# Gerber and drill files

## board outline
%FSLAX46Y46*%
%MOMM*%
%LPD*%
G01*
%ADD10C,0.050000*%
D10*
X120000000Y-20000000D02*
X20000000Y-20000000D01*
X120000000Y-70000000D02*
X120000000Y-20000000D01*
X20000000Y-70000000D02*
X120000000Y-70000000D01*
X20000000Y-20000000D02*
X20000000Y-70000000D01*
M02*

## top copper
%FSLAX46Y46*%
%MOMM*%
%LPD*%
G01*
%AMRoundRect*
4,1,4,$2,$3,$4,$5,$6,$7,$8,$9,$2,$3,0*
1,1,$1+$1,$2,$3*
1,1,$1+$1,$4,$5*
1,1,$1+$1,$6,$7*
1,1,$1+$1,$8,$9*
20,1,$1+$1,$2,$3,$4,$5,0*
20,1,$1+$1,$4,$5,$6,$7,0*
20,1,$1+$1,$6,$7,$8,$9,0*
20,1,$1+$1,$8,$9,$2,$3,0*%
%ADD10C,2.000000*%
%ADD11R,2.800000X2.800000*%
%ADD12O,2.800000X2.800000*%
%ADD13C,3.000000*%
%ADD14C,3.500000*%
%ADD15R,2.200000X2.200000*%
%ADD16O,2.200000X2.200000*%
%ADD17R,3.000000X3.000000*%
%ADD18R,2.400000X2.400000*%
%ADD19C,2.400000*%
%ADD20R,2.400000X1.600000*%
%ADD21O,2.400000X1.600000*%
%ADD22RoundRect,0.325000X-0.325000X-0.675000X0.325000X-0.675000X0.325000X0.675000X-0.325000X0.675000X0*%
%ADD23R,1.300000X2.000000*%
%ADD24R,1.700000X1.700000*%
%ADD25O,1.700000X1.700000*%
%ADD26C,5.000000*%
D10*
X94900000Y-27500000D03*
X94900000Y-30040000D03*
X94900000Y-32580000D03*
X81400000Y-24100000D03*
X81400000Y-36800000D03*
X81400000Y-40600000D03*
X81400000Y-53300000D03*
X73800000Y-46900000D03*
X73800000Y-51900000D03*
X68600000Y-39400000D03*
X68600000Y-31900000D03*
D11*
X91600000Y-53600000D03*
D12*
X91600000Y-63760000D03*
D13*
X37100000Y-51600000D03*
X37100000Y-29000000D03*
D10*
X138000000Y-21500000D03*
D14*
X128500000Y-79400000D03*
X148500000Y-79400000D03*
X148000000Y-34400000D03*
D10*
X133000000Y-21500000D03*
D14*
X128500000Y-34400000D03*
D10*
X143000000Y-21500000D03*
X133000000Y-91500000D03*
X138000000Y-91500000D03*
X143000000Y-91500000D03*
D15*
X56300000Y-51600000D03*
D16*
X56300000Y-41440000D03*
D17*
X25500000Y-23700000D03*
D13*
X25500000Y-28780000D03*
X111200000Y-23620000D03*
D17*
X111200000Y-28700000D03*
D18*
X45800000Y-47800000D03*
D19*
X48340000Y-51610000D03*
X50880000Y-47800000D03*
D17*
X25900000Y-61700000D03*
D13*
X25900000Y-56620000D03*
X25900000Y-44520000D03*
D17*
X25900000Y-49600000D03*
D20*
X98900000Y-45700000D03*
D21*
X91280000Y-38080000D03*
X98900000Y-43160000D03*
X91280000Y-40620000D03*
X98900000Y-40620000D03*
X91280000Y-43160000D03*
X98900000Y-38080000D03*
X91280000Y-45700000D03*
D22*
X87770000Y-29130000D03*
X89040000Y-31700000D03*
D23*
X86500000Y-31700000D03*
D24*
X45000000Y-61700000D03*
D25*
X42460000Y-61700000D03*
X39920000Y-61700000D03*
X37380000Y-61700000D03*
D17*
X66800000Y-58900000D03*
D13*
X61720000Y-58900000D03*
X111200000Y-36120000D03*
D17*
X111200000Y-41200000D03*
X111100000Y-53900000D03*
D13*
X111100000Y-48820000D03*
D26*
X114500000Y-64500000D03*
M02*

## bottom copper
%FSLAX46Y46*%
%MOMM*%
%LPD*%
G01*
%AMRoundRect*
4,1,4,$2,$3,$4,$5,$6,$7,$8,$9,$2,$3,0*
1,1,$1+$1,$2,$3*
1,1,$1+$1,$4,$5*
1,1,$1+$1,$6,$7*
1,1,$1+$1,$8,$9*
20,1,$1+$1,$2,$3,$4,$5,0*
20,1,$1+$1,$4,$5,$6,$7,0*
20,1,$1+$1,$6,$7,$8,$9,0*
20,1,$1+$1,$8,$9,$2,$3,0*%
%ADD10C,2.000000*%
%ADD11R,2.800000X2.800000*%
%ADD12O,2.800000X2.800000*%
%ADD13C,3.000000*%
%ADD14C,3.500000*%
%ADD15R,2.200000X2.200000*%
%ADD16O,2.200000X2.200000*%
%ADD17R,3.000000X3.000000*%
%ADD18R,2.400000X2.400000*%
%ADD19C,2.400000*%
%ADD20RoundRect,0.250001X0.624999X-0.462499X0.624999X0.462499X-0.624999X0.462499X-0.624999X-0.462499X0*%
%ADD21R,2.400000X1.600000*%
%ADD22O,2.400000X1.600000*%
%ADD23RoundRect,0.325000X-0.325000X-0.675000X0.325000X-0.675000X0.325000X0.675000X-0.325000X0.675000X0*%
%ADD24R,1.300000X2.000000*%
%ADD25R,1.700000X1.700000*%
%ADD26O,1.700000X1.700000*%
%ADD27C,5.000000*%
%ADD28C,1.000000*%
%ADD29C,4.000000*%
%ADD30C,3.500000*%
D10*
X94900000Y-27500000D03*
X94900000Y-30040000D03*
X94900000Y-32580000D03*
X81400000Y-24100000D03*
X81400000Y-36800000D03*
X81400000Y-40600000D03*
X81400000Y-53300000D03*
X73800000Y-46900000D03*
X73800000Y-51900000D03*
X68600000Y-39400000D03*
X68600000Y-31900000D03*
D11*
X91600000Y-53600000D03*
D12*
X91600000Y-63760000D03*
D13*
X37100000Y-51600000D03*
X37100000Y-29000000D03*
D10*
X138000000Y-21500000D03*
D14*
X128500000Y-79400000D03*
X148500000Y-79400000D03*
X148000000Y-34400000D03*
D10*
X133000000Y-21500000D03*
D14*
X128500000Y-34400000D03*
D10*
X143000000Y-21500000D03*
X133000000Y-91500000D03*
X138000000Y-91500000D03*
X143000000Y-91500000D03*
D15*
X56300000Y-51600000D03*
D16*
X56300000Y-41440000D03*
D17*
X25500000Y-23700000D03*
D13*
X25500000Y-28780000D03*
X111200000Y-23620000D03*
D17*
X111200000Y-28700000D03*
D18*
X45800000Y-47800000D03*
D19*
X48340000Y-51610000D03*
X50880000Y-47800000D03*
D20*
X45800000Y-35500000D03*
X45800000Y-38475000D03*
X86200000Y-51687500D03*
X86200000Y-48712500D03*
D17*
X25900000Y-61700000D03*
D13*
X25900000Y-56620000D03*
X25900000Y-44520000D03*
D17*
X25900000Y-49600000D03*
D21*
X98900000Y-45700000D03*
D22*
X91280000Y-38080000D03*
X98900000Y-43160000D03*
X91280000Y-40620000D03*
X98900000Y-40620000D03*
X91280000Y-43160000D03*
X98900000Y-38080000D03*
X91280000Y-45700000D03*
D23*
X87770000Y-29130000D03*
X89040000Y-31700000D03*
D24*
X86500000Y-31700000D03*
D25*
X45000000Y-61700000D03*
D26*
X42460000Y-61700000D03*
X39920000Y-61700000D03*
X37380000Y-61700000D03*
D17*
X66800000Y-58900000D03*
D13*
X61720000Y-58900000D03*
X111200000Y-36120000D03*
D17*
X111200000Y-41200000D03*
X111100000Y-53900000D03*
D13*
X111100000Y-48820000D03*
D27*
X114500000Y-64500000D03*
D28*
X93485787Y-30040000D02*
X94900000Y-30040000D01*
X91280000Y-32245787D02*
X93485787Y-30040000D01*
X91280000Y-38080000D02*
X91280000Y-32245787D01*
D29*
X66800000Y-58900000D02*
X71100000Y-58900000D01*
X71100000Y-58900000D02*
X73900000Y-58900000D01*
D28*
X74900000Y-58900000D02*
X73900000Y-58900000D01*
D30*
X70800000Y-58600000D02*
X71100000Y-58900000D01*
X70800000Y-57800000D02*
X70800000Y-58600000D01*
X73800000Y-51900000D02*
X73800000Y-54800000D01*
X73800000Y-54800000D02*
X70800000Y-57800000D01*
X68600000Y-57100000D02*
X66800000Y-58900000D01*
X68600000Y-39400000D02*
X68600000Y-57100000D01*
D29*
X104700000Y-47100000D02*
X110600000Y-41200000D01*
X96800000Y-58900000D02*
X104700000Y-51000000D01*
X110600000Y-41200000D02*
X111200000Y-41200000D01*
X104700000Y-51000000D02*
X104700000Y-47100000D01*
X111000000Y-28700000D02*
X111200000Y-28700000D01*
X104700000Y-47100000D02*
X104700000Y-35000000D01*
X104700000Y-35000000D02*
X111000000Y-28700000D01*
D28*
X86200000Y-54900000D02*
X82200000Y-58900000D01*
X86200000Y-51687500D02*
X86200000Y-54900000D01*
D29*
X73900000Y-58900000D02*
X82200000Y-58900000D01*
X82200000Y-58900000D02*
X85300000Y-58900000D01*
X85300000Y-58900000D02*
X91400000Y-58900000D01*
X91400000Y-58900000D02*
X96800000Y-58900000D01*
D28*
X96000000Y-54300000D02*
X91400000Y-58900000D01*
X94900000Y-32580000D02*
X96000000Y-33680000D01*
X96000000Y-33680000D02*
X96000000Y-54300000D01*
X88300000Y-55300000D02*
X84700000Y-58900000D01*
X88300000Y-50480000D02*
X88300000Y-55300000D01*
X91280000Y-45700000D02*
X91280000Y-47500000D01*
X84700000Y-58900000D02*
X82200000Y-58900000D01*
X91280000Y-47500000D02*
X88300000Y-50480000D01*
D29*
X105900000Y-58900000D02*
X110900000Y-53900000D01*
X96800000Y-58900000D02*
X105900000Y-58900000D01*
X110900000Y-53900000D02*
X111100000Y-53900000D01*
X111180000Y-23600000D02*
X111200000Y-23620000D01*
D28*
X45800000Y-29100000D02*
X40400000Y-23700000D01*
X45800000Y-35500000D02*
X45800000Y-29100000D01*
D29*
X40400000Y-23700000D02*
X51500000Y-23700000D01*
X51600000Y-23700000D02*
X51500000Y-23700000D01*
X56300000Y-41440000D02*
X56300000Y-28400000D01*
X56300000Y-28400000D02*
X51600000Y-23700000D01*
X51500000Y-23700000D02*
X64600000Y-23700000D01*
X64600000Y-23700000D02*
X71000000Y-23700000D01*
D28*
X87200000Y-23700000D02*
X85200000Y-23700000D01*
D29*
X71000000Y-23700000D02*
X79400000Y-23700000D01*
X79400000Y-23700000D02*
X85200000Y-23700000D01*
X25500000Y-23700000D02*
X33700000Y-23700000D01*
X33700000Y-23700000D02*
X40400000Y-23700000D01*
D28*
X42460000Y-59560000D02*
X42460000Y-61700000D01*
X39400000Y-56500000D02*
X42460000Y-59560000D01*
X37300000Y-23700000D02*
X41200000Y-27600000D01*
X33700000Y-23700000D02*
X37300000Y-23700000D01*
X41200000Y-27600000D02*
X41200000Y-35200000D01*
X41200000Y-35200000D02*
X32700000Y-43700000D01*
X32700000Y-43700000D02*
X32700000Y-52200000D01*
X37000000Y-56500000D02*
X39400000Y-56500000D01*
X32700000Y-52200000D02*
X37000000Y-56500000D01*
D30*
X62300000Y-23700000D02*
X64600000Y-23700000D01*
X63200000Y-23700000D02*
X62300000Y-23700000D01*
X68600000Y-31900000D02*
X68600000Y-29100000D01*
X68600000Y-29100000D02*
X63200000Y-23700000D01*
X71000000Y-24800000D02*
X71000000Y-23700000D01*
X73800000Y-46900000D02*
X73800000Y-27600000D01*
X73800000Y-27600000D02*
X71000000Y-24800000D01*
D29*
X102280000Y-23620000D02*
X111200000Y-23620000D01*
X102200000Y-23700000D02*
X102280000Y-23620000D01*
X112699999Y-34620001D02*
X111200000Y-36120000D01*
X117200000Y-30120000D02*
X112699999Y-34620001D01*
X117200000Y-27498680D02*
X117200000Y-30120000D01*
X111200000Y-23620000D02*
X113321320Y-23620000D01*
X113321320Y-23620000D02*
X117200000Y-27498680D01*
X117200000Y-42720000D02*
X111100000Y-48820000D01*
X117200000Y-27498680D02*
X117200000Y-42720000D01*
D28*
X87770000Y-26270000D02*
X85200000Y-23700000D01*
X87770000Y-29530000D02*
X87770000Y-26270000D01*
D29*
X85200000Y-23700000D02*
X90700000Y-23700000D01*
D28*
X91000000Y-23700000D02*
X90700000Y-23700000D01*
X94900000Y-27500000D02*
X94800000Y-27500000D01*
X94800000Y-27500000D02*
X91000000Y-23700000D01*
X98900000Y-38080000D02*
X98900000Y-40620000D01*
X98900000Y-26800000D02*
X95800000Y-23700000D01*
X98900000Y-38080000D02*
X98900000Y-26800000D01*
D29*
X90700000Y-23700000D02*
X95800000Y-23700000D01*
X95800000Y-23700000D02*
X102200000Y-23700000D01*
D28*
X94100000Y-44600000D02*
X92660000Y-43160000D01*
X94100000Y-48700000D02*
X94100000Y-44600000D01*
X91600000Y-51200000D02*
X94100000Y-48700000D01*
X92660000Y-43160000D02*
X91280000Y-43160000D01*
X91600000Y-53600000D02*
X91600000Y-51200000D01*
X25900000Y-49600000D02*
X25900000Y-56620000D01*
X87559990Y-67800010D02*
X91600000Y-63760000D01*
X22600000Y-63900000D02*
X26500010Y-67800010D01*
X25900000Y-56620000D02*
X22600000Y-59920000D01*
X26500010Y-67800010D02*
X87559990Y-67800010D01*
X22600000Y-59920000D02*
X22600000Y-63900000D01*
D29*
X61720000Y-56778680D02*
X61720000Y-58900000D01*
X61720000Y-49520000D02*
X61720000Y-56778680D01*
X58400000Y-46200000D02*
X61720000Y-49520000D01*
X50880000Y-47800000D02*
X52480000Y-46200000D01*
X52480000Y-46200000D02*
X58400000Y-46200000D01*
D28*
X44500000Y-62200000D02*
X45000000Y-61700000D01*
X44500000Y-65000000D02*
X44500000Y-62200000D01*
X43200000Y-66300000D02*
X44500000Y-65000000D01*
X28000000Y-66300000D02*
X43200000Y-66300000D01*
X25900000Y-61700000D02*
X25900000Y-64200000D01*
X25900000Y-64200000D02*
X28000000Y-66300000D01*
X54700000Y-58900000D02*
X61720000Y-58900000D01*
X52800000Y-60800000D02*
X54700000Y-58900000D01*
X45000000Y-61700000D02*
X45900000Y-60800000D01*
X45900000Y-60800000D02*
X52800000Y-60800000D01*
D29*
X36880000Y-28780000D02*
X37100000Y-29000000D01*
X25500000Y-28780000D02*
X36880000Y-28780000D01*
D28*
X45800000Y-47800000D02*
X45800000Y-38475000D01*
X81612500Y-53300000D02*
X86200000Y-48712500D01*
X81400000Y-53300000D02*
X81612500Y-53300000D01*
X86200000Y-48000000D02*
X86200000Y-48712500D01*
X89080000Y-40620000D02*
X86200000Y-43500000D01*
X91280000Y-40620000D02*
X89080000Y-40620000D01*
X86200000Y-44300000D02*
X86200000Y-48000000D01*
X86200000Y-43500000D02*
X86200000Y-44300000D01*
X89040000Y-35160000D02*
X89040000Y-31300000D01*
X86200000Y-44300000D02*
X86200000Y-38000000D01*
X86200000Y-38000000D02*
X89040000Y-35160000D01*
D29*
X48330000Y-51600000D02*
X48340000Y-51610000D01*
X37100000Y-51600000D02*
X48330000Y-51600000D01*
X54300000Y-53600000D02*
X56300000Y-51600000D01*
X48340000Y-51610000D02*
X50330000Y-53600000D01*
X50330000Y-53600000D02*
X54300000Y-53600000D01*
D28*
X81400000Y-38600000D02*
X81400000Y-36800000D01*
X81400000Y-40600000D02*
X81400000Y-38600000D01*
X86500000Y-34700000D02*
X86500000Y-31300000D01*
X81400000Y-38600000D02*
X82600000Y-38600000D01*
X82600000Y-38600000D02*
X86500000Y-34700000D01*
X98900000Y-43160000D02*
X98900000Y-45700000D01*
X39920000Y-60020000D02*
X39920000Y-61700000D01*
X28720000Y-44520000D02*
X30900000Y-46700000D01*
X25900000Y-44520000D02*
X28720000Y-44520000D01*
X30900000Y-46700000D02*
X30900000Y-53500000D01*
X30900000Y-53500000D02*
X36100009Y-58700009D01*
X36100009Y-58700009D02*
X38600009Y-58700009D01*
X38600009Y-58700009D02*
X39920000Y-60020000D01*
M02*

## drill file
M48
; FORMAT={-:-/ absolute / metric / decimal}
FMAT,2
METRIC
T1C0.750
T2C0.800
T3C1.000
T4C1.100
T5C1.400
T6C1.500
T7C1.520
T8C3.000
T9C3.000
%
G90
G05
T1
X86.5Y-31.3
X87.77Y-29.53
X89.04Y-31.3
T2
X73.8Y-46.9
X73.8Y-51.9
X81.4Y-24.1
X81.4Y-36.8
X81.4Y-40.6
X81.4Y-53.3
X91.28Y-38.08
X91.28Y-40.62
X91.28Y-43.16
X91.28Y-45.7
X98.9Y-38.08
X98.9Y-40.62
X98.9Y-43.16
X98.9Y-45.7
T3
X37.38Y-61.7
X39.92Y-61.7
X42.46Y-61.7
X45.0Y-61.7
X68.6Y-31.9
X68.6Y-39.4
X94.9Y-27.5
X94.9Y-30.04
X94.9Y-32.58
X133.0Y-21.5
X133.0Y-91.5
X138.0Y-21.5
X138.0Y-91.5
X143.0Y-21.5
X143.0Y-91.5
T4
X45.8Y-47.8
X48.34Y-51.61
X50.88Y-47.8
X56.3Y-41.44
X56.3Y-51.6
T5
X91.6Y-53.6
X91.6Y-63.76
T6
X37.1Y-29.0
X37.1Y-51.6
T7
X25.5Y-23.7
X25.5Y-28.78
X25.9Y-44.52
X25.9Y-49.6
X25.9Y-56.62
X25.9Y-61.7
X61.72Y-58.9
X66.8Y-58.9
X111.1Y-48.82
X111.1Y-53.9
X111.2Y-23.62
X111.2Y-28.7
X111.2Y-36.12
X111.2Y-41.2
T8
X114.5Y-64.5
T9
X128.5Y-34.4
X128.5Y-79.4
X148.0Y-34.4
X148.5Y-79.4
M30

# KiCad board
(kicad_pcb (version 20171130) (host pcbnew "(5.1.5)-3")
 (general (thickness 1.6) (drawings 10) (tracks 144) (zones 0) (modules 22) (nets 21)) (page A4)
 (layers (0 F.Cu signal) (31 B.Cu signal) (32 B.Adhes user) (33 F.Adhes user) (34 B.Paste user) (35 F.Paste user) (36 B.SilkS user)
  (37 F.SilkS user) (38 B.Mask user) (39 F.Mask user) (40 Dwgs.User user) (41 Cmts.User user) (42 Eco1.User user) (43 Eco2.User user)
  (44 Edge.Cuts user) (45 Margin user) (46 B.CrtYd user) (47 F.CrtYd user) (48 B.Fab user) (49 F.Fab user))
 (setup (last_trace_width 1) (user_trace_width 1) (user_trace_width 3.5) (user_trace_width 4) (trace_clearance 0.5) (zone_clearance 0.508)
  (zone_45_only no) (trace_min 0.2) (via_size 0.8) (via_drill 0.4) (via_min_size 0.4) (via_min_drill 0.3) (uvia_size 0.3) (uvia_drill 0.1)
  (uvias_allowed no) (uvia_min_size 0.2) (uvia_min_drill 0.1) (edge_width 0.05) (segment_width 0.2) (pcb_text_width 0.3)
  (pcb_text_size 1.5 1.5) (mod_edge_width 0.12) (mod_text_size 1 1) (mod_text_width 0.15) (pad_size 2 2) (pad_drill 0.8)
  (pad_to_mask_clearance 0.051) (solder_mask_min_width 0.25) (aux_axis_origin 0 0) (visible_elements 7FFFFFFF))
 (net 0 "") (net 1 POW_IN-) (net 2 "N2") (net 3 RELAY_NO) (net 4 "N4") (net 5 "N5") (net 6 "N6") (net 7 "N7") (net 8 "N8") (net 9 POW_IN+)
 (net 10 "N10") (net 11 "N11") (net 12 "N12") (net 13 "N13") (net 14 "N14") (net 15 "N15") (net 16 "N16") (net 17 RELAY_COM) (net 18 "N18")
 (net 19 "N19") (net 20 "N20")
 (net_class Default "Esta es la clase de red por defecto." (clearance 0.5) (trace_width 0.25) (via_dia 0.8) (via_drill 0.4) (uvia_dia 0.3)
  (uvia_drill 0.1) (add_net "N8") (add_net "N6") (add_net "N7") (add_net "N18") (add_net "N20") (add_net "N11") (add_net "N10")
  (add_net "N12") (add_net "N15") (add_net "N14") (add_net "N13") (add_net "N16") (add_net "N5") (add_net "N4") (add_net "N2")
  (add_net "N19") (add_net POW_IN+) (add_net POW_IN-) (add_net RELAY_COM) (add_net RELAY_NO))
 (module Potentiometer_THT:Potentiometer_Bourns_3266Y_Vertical (layer F.Cu) (at 94.9 27.5 90)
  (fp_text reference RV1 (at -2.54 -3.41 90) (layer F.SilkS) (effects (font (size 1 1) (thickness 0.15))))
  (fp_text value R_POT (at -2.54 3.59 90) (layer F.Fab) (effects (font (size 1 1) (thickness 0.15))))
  (pad 1 thru_hole circle (at 0 0 90) (size 2 2) (drill 1) (layers *.Cu *.Mask) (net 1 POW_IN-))
  (pad 2 thru_hole circle (at -2.54 0 90) (size 2 2) (drill 1) (layers *.Cu *.Mask) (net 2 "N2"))
  (pad 3 thru_hole circle (at -5.08 0 90) (size 2 2) (drill 1) (layers *.Cu *.Mask) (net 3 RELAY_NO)))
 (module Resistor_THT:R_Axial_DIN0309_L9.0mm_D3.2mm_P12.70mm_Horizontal (layer F.Cu) (at 81.4 36.8 90)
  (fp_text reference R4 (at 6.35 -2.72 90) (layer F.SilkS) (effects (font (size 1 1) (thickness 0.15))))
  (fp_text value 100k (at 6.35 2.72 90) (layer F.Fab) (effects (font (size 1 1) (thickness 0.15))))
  (pad 2 thru_hole circle (at 12.7 0 90) (size 2 2) (drill 0.8) (layers *.Cu *.Mask) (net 1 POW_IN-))
  (pad 1 thru_hole circle (at 0 0 90) (size 2 2) (drill 0.8) (layers *.Cu *.Mask) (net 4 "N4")))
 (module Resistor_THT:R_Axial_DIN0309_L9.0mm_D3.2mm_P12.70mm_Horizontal (layer F.Cu) (at 81.4 53.3 90)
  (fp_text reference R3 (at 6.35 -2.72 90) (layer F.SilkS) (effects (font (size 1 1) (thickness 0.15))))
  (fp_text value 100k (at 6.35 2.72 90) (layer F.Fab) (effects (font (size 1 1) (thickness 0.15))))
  (pad 2 thru_hole circle (at 12.7 0 90) (size 2 2) (drill 0.8) (layers *.Cu *.Mask) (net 4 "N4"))
  (pad 1 thru_hole circle (at 0 0 90) (size 2 2) (drill 0.8) (layers *.Cu *.Mask) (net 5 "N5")))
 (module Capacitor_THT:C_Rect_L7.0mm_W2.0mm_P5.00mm (layer B.Cu) (at 73.8 51.9 90)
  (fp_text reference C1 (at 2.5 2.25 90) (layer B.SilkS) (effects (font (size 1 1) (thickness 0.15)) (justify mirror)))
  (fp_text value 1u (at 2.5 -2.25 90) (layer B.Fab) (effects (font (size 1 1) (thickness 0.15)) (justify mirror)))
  (pad 2 thru_hole circle (at 5 0 90) (size 2 2) (drill 0.8) (layers *.Cu *.Mask) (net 1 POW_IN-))
  (pad 1 thru_hole circle (at 0 0 90) (size 2 2) (drill 0.8) (layers *.Cu *.Mask) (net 3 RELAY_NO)))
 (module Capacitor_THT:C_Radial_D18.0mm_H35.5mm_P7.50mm (layer F.Cu) (at 68.6 39.4 90)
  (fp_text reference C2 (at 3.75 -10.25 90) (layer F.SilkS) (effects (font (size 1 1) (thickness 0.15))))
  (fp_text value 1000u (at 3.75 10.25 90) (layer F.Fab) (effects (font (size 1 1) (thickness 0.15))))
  (pad 1 thru_hole circle (at 0 0 90) (size 2 2) (drill 1) (layers *.Cu *.Mask) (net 3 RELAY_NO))
  (pad 2 thru_hole circle (at 7.5 0 90) (size 2 2) (drill 1) (layers *.Cu *.Mask) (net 1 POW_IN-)))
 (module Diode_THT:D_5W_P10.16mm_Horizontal (layer F.Cu) (at 91.6 53.6 270)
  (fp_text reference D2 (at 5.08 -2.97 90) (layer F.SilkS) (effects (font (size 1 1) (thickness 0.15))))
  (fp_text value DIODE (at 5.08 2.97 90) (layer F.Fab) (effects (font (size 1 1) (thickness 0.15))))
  (pad 1 thru_hole rect (at 0 0 270) (size 2.8 2.8) (drill 1.4) (layers *.Cu *.Mask) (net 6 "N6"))
  (pad 2 thru_hole oval (at 10.16 0 270) (size 2.8 2.8) (drill 1.4) (layers *.Cu *.Mask) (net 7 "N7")))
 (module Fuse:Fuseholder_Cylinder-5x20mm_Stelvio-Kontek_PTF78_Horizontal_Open (layer F.Cu) (at 37.1 51.6 90)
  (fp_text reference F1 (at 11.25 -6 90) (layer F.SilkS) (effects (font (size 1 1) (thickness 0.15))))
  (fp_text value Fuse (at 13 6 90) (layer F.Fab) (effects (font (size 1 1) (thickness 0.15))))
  (pad 1 thru_hole circle (at 0 0 90) (size 3 3) (drill 1.5) (layers *.Cu *.Mask) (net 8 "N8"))
  (pad 2 thru_hole circle (at 22.6 0 90) (size 3 3) (drill 1.5) (layers *.Cu *.Mask) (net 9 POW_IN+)))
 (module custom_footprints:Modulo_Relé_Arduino (layer F.Cu) (at 128.5 34.4 90)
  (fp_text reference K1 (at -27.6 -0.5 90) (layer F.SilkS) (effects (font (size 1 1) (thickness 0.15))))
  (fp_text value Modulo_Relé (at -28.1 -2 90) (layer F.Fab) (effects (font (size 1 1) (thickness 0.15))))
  (pad 2 thru_hole circle (at 12.9 9.5 90) (size 2 2) (drill 1) (layers *.Cu *.Mask) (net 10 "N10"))
  (pad "" np_thru_hole circle (at -45 0 90) (size 3.5 3.5) (drill 3) (layers *.Cu *.Mask))
  (pad "" np_thru_hole circle (at -45 20 90) (size 3.5 3.5) (drill 3) (layers *.Cu *.Mask))
  (pad "" np_thru_hole circle (at 0 19.5 90) (size 3.5 3.5) (drill 3) (layers *.Cu *.Mask))
  (pad 1 thru_hole circle (at 12.9 4.5 90) (size 2 2) (drill 1) (layers *.Cu *.Mask) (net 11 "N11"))
  (pad "" np_thru_hole circle (at 0 0 90) (size 3.5 3.5) (drill 3) (layers *.Cu *.Mask))
  (pad 3 thru_hole circle (at 12.9 14.5 90) (size 2 2) (drill 1) (layers *.Cu *.Mask) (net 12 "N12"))
  (pad 6 thru_hole circle (at -57.1 4.5 90) (size 2 2) (drill 1) (layers *.Cu *.Mask) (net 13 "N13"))
  (pad 5 thru_hole circle (at -57.1 9.5 90) (size 2 2) (drill 1) (layers *.Cu *.Mask) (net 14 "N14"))
  (pad 4 thru_hole circle (at -57.1 14.5 90) (size 2 2) (drill 1) (layers *.Cu *.Mask) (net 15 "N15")))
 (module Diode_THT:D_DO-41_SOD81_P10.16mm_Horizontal (layer F.Cu) (at 56.3 51.6 90)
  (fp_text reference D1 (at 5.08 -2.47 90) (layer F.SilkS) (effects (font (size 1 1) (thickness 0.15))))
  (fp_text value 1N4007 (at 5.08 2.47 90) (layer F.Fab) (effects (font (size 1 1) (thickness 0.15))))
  (pad 1 thru_hole rect (at 0 0 90) (size 2.2 2.2) (drill 1.1) (layers *.Cu *.Mask) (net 8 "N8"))
  (pad 2 thru_hole oval (at 10.16 0 90) (size 2.2 2.2) (drill 1.1) (layers *.Cu *.Mask) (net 1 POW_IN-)))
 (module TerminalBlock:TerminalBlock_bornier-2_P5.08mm (layer F.Cu) (at 25.5 23.7 270)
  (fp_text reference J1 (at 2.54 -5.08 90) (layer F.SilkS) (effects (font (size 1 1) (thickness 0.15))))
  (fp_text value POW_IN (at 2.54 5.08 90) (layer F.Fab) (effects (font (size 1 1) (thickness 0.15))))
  (pad 1 thru_hole rect (at 0 0 270) (size 3 3) (drill 1.52) (layers *.Cu *.Mask) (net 1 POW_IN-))
  (pad 2 thru_hole circle (at 5.08 0 270) (size 3 3) (drill 1.52) (layers *.Cu *.Mask) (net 9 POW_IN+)))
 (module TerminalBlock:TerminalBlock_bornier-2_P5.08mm (layer F.Cu) (at 111.2 28.7 90)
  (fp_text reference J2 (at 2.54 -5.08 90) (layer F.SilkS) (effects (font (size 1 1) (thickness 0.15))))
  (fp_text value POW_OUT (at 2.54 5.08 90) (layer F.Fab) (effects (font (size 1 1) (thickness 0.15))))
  (pad 2 thru_hole circle (at 5.08 0 90) (size 3 3) (drill 1.52) (layers *.Cu *.Mask) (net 1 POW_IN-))
  (pad 1 thru_hole rect (at 0 0 90) (size 3 3) (drill 1.52) (layers *.Cu *.Mask) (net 3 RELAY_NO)))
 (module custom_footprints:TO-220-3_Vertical (layer F.Cu) (at 45.8 47.8)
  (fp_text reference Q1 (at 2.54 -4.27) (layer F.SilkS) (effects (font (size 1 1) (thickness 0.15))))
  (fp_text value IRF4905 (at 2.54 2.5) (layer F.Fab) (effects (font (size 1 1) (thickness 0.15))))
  (pad 1 thru_hole rect (at 0 0) (size 2.4 2.4) (drill 1.1) (layers *.Cu *.Mask) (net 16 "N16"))
  (pad 2 thru_hole circle (at 2.54 3.81) (size 2.4 2.4) (drill 1.1) (layers *.Cu *.Mask) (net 8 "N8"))
  (pad 3 thru_hole circle (at 5.08 0) (size 2.4 2.4) (drill 1.1) (layers *.Cu *.Mask) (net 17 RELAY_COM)))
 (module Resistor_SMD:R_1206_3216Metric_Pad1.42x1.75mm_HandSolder (layer B.Cu) (at 45.8 36.9875 90)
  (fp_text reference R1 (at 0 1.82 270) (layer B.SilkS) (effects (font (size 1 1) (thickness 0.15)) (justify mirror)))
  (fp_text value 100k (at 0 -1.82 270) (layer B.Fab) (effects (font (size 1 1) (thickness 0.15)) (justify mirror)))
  (pad 2 smd roundrect (at 1.4875 0 90) (size 1.425 1.75) (layers B.Cu B.Paste B.Mask) (roundrect_rratio 0.175439) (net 1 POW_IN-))
  (pad 1 smd roundrect (at -1.4875 0 90) (size 1.425 1.75) (layers B.Cu B.Paste B.Mask) (roundrect_rratio 0.175439) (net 16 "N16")))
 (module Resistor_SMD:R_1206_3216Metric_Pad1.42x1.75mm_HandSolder (layer B.Cu) (at 86.2 50.2 90)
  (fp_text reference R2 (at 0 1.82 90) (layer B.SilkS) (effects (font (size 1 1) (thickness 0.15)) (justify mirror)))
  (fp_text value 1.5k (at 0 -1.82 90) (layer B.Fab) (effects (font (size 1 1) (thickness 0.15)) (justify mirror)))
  (pad 1 smd roundrect (at -1.4875 0 90) (size 1.425 1.75) (layers B.Cu B.Paste B.Mask) (roundrect_rratio 0.175439) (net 3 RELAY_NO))
  (pad 2 smd roundrect (at 1.4875 0 90) (size 1.425 1.75) (layers B.Cu B.Paste B.Mask) (roundrect_rratio 0.175439) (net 5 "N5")))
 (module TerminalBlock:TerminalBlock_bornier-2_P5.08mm (layer F.Cu) (at 25.9 61.7 90)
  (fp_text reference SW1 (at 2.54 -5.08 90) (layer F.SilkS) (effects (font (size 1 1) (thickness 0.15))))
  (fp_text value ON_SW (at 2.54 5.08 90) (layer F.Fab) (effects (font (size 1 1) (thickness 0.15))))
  (pad 1 thru_hole rect (at 0 0 90) (size 3 3) (drill 1.52) (layers *.Cu *.Mask) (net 17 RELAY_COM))
  (pad 2 thru_hole circle (at 5.08 0 90) (size 3 3) (drill 1.52) (layers *.Cu *.Mask) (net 7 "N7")))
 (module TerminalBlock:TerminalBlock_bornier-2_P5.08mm (layer F.Cu) (at 25.9 49.6 90)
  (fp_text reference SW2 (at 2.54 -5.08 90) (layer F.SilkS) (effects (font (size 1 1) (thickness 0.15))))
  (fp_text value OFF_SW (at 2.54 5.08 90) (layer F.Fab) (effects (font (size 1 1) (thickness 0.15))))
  (pad 2 thru_hole circle (at 5.08 0 90) (size 3 3) (drill 1.52) (layers *.Cu *.Mask) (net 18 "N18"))
  (pad 1 thru_hole rect (at 0 0 90) (size 3 3) (drill 1.52) (layers *.Cu *.Mask) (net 7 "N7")))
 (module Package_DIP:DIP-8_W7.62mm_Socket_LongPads (layer F.Cu) (at 98.9 45.7 180)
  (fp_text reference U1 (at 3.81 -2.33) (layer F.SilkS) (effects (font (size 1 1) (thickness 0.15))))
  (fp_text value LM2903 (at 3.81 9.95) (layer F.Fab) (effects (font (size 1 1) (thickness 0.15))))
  (pad 1 thru_hole rect (at 0 0 180) (size 2.4 1.6) (drill 0.8) (layers *.Cu *.Mask) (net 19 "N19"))
  (pad 5 thru_hole oval (at 7.62 7.62 180) (size 2.4 1.6) (drill 0.8) (layers *.Cu *.Mask) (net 2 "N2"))
  (pad 2 thru_hole oval (at 0 2.54 180) (size 2.4 1.6) (drill 0.8) (layers *.Cu *.Mask) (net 19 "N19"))
  (pad 6 thru_hole oval (at 7.62 5.08 180) (size 2.4 1.6) (drill 0.8) (layers *.Cu *.Mask) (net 5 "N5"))
  (pad 3 thru_hole oval (at 0 5.08 180) (size 2.4 1.6) (drill 0.8) (layers *.Cu *.Mask) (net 1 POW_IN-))
  (pad 7 thru_hole oval (at 7.62 2.54 180) (size 2.4 1.6) (drill 0.8) (layers *.Cu *.Mask) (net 6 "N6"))
  (pad 4 thru_hole oval (at 0 7.62 180) (size 2.4 1.6) (drill 0.8) (layers *.Cu *.Mask) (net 1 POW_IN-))
  (pad 8 thru_hole oval (at 7.62 0 180) (size 2.4 1.6) (drill 0.8) (layers *.Cu *.Mask) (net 3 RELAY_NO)))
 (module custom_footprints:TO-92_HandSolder (layer F.Cu) (at 86.5 30.8)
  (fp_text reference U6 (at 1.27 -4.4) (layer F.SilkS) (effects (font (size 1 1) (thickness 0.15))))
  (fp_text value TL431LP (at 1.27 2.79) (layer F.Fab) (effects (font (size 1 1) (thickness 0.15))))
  (pad 2 thru_hole roundrect (at 1.27 -1.27) (size 1.3 2) (drill 0.75 (offset 0 -0.4)) (layers *.Cu *.Mask) (roundrect_rratio 0.25)
   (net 1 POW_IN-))
  (pad 3 thru_hole roundrect (at 2.54 0.5) (size 1.3 2) (drill 0.75 (offset 0 0.4)) (layers *.Cu *.Mask) (roundrect_rratio 0.25)
   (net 5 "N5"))
  (pad 1 thru_hole rect (at 0 0.5) (size 1.3 2) (drill 0.75 (offset 0 0.4)) (layers *.Cu *.Mask) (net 4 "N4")))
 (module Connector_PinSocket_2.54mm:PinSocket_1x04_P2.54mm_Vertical (layer F.Cu) (at 45 61.7 270)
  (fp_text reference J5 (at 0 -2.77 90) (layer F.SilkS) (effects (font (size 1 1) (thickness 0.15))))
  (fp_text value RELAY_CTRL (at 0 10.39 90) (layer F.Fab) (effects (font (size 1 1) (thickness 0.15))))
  (pad 1 thru_hole rect (at 0 0 270) (size 1.7 1.7) (drill 1) (layers *.Cu *.Mask) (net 17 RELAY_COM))
  (pad 2 thru_hole oval (at 0 2.54 270) (size 1.7 1.7) (drill 1) (layers *.Cu *.Mask) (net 1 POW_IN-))
  (pad 3 thru_hole oval (at 0 5.08 270) (size 1.7 1.7) (drill 1) (layers *.Cu *.Mask) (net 18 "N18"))
  (pad 4 thru_hole oval (at 0 7.62 270) (size 1.7 1.7) (drill 1) (layers *.Cu *.Mask) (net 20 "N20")))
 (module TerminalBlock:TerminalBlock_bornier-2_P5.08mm (layer F.Cu) (at 66.8 58.9 180)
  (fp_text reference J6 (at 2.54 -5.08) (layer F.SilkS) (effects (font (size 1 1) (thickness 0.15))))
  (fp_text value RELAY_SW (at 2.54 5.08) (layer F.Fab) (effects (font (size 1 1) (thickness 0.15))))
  (pad 1 thru_hole rect (at 0 0 180) (size 3 3) (drill 1.52) (layers *.Cu *.Mask) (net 3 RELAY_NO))
  (pad 2 thru_hole circle (at 5.08 0 180) (size 3 3) (drill 1.52) (layers *.Cu *.Mask) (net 17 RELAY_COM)))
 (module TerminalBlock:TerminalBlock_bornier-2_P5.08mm (layer F.Cu) (at 111.2 41.2 90)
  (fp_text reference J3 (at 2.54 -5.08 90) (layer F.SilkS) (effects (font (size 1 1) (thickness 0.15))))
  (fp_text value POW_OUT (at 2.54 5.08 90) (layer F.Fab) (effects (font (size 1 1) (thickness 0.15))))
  (pad 2 thru_hole circle (at 5.08 0 90) (size 3 3) (drill 1.52) (layers *.Cu *.Mask) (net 1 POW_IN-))
  (pad 1 thru_hole rect (at 0 0 90) (size 3 3) (drill 1.52) (layers *.Cu *.Mask) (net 3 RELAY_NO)))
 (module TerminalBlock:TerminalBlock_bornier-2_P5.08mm (layer F.Cu) (at 111.1 53.9 90)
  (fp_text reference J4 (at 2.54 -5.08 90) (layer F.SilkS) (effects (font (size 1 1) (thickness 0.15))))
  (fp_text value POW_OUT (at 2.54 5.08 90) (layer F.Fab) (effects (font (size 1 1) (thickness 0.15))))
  (pad 1 thru_hole rect (at 0 0 90) (size 3 3) (drill 1.52) (layers *.Cu *.Mask) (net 3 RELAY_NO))
  (pad 2 thru_hole circle (at 5.08 0 90) (size 3 3) (drill 1.52) (layers *.Cu *.Mask) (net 1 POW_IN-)))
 (gr_line (start 120 20) (end 20 20) (layer Edge.Cuts) (width 0.05))
 (gr_line (start 120 70) (end 120 20) (layer Edge.Cuts) (width 0.05))
 (gr_line (start 20 70) (end 120 70) (layer Edge.Cuts) (width 0.05))
 (gr_line (start 20 20) (end 20 70) (layer Edge.Cuts) (width 0.05))
 (via (at 114.5 64.5) (size 5) (drill 3) (layers F.Cu B.Cu) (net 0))
 (segment (start 93.485787 30.04) (end 94.9 30.04) (width 1) (layer B.Cu) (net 2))
 (segment (start 91.28 32.245787) (end 93.485787 30.04) (width 1) (layer B.Cu) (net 2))
 (segment (start 91.28 38.08) (end 91.28 32.245787) (width 1) (layer B.Cu) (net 2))
 (segment (start 66.8 58.9) (end 71.1 58.9) (width 4) (layer B.Cu) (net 3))
 (segment (start 71.1 58.9) (end 73.9 58.9) (width 4) (layer B.Cu) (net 3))
 (segment (start 74.9 58.9) (end 73.9 58.9) (width 1) (layer B.Cu) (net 3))
 (segment (start 70.8 58.6) (end 71.1 58.9) (width 3.5) (layer B.Cu) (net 3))
 (segment (start 70.8 57.8) (end 70.8 58.6) (width 3.5) (layer B.Cu) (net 3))
 (segment (start 73.8 51.9) (end 73.8 54.8) (width 3.5) (layer B.Cu) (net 3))
 (segment (start 73.8 54.8) (end 70.8 57.8) (width 3.5) (layer B.Cu) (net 3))
 (segment (start 68.6 57.1) (end 66.8 58.9) (width 3.5) (layer B.Cu) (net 3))
 (segment (start 68.6 39.4) (end 68.6 57.1) (width 3.5) (layer B.Cu) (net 3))
 (segment (start 104.7 47.1) (end 110.6 41.2) (width 4) (layer B.Cu) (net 3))
 (segment (start 96.8 58.9) (end 104.7 51) (width 4) (layer B.Cu) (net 3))
 (segment (start 110.6 41.2) (end 111.2 41.2) (width 4) (layer B.Cu) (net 3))
 (segment (start 104.7 51) (end 104.7 47.1) (width 4) (layer B.Cu) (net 3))
 (segment (start 111 28.7) (end 111.2 28.7) (width 4) (layer B.Cu) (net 3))
 (segment (start 104.7 47.1) (end 104.7 35) (width 4) (layer B.Cu) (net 3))
 (segment (start 104.7 35) (end 111 28.7) (width 4) (layer B.Cu) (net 3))
 (segment (start 86.2 54.9) (end 82.2 58.9) (width 1) (layer B.Cu) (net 3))
 (segment (start 86.2 51.6875) (end 86.2 54.9) (width 1) (layer B.Cu) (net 3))
 (segment (start 73.9 58.9) (end 82.2 58.9) (width 4) (layer B.Cu) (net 3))
 (segment (start 82.2 58.9) (end 85.3 58.9) (width 4) (layer B.Cu) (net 3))
 (segment (start 85.3 58.9) (end 91.4 58.9) (width 4) (layer B.Cu) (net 3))
 (segment (start 91.4 58.9) (end 96.8 58.9) (width 4) (layer B.Cu) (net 3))
 (segment (start 96 54.3) (end 91.4 58.9) (width 1) (layer B.Cu) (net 3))
 (segment (start 94.9 32.58) (end 96 33.68) (width 1) (layer B.Cu) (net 3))
 (segment (start 96 33.68) (end 96 54.3) (width 1) (layer B.Cu) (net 3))
 (segment (start 88.3 55.3) (end 84.7 58.9) (width 1) (layer B.Cu) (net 3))
 (segment (start 88.3 50.48) (end 88.3 55.3) (width 1) (layer B.Cu) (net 3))
 (segment (start 91.28 45.7) (end 91.28 47.5) (width 1) (layer B.Cu) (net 3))
 (segment (start 84.7 58.9) (end 82.2 58.9) (width 1) (layer B.Cu) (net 3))
 (segment (start 91.28 47.5) (end 88.3 50.48) (width 1) (layer B.Cu) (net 3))
 (segment (start 105.9 58.9) (end 110.9 53.9) (width 4) (layer B.Cu) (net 3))
 (segment (start 96.8 58.9) (end 105.9 58.9) (width 4) (layer B.Cu) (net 3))
 (segment (start 110.9 53.9) (end 111.1 53.9) (width 4) (layer B.Cu) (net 3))
 (segment (start 111.18 23.6) (end 111.2 23.62) (width 4) (layer B.Cu) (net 1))
 (segment (start 45.8 29.1) (end 40.4 23.7) (width 1) (layer B.Cu) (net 1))
 (segment (start 45.8 35.5) (end 45.8 29.1) (width 1) (layer B.Cu) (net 1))
 (segment (start 40.4 23.7) (end 51.5 23.7) (width 4) (layer B.Cu) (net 1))
 (segment (start 51.6 23.7) (end 51.5 23.7) (width 4) (layer B.Cu) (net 1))
 (segment (start 56.3 41.44) (end 56.3 28.4) (width 4) (layer B.Cu) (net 1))
 (segment (start 56.3 28.4) (end 51.6 23.7) (width 4) (layer B.Cu) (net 1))
 (segment (start 51.5 23.7) (end 64.6 23.7) (width 4) (layer B.Cu) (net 1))
 (segment (start 64.6 23.7) (end 71 23.7) (width 4) (layer B.Cu) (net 1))
 (segment (start 87.2 23.7) (end 85.2 23.7) (width 1) (layer B.Cu) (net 1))
 (segment (start 71 23.7) (end 79.4 23.7) (width 4) (layer B.Cu) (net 1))
 (segment (start 79.4 23.7) (end 85.2 23.7) (width 4) (layer B.Cu) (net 1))
 (segment (start 25.5 23.7) (end 33.7 23.7) (width 4) (layer B.Cu) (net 1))
 (segment (start 33.7 23.7) (end 40.4 23.7) (width 4) (layer B.Cu) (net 1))
 (segment (start 42.46 59.56) (end 42.46 61.7) (width 1) (layer B.Cu) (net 1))
 (segment (start 39.4 56.5) (end 42.46 59.56) (width 1) (layer B.Cu) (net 1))
 (segment (start 37.3 23.7) (end 41.2 27.6) (width 1) (layer B.Cu) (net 1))
 (segment (start 33.7 23.7) (end 37.3 23.7) (width 1) (layer B.Cu) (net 1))
 (segment (start 41.2 27.6) (end 41.2 35.2) (width 1) (layer B.Cu) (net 1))
 (segment (start 41.2 35.2) (end 32.7 43.7) (width 1) (layer B.Cu) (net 1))
 (segment (start 32.7 43.7) (end 32.7 52.2) (width 1) (layer B.Cu) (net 1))
 (segment (start 37 56.5) (end 39.4 56.5) (width 1) (layer B.Cu) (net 1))
 (segment (start 32.7 52.2) (end 37 56.5) (width 1) (layer B.Cu) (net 1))
 (segment (start 62.3 23.7) (end 64.6 23.7) (width 3.5) (layer B.Cu) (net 1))
 (segment (start 63.2 23.7) (end 62.3 23.7) (width 3.5) (layer B.Cu) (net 1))
 (segment (start 68.6 31.9) (end 68.6 29.1) (width 3.5) (layer B.Cu) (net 1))
 (segment (start 68.6 29.1) (end 63.2 23.7) (width 3.5) (layer B.Cu) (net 1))
 (segment (start 71 24.8) (end 71 23.7) (width 3.5) (layer B.Cu) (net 1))
 (segment (start 73.8 46.9) (end 73.8 27.6) (width 3.5) (layer B.Cu) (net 1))
 (segment (start 73.8 27.6) (end 71 24.8) (width 3.5) (layer B.Cu) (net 1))
 (segment (start 102.28 23.62) (end 111.2 23.62) (width 4) (layer B.Cu) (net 1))
 (segment (start 102.2 23.7) (end 102.28 23.62) (width 4) (layer B.Cu) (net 1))
 (segment (start 112.699999 34.620001) (end 111.2 36.12) (width 4) (layer B.Cu) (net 1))
 (segment (start 117.2 30.12) (end 112.699999 34.620001) (width 4) (layer B.Cu) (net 1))
 (segment (start 117.2 27.49868) (end 117.2 30.12) (width 4) (layer B.Cu) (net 1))
 (segment (start 111.2 23.62) (end 113.32132 23.62) (width 4) (layer B.Cu) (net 1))
 (segment (start 113.32132 23.62) (end 117.2 27.49868) (width 4) (layer B.Cu) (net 1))
 (segment (start 117.2 42.72) (end 111.1 48.82) (width 4) (layer B.Cu) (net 1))
 (segment (start 117.2 27.49868) (end 117.2 42.72) (width 4) (layer B.Cu) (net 1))
 (segment (start 87.77 26.27) (end 85.2 23.7) (width 1) (layer B.Cu) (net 1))
 (segment (start 87.77 29.53) (end 87.77 26.27) (width 1) (layer B.Cu) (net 1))
 (segment (start 85.2 23.7) (end 90.7 23.7) (width 4) (layer B.Cu) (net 1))
 (segment (start 91 23.7) (end 90.7 23.7) (width 1) (layer B.Cu) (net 1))
 (segment (start 94.9 27.5) (end 94.8 27.5) (width 1) (layer B.Cu) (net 1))
 (segment (start 94.8 27.5) (end 91 23.7) (width 1) (layer B.Cu) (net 1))
 (segment (start 98.9 38.08) (end 98.9 40.62) (width 1) (layer B.Cu) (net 1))
 (segment (start 98.9 26.8) (end 95.8 23.7) (width 1) (layer B.Cu) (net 1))
 (segment (start 98.9 38.08) (end 98.9 26.8) (width 1) (layer B.Cu) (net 1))
 (segment (start 90.7 23.7) (end 95.8 23.7) (width 4) (layer B.Cu) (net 1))
 (segment (start 95.8 23.7) (end 102.2 23.7) (width 4) (layer B.Cu) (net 1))
 (segment (start 94.1 44.6) (end 92.66 43.16) (width 1) (layer B.Cu) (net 6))
 (segment (start 94.1 48.7) (end 94.1 44.6) (width 1) (layer B.Cu) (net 6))
 (segment (start 91.6 51.2) (end 94.1 48.7) (width 1) (layer B.Cu) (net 6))
 (segment (start 92.66 43.16) (end 91.28 43.16) (width 1) (layer B.Cu) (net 6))
 (segment (start 91.6 53.6) (end 91.6 51.2) (width 1) (layer B.Cu) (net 6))
 (segment (start 25.9 49.6) (end 25.9 56.62) (width 1) (layer B.Cu) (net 7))
 (segment (start 87.55999 67.80001) (end 91.6 63.76) (width 1) (layer B.Cu) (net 7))
 (segment (start 22.6 63.9) (end 26.50001 67.80001) (width 1) (layer B.Cu) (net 7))
 (segment (start 25.9 56.62) (end 22.6 59.92) (width 1) (layer B.Cu) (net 7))
 (segment (start 26.50001 67.80001) (end 87.55999 67.80001) (width 1) (layer B.Cu) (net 7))
 (segment (start 22.6 59.92) (end 22.6 63.9) (width 1) (layer B.Cu) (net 7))
 (segment (start 61.72 56.77868) (end 61.72 58.9) (width 4) (layer B.Cu) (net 17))
 (segment (start 61.72 49.52) (end 61.72 56.77868) (width 4) (layer B.Cu) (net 17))
 (segment (start 58.4 46.2) (end 61.72 49.52) (width 4) (layer B.Cu) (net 17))
 (segment (start 50.88 47.8) (end 52.48 46.2) (width 4) (layer B.Cu) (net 17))
 (segment (start 52.48 46.2) (end 58.4 46.2) (width 4) (layer B.Cu) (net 17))
 (segment (start 44.5 62.2) (end 45 61.7) (width 1) (layer B.Cu) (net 17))
 (segment (start 44.5 65) (end 44.5 62.2) (width 1) (layer B.Cu) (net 17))
 (segment (start 43.2 66.3) (end 44.5 65) (width 1) (layer B.Cu) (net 17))
 (segment (start 28 66.3) (end 43.2 66.3) (width 1) (layer B.Cu) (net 17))
 (segment (start 25.9 61.7) (end 25.9 64.2) (width 1) (layer B.Cu) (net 17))
 (segment (start 25.9 64.2) (end 28 66.3) (width 1) (layer B.Cu) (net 17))
 (segment (start 54.7 58.9) (end 61.72 58.9) (width 1) (layer B.Cu) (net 17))
 (segment (start 52.8 60.8) (end 54.7 58.9) (width 1) (layer B.Cu) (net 17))
 (segment (start 45 61.7) (end 45.9 60.8) (width 1) (layer B.Cu) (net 17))
 (segment (start 45.9 60.8) (end 52.8 60.8) (width 1) (layer B.Cu) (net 17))
 (segment (start 36.88 28.78) (end 37.1 29) (width 4) (layer B.Cu) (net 9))
 (segment (start 25.5 28.78) (end 36.88 28.78) (width 4) (layer B.Cu) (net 9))
 (segment (start 45.8 47.8) (end 45.8 38.475) (width 1) (layer B.Cu) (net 16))
 (segment (start 81.6125 53.3) (end 86.2 48.7125) (width 1) (layer B.Cu) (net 5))
 (segment (start 81.4 53.3) (end 81.6125 53.3) (width 1) (layer B.Cu) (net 5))
 (segment (start 86.2 48) (end 86.2 48.7125) (width 1) (layer B.Cu) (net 5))
 (segment (start 89.08 40.62) (end 86.2 43.5) (width 1) (layer B.Cu) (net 5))
 (segment (start 91.28 40.62) (end 89.08 40.62) (width 1) (layer B.Cu) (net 5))
 (segment (start 86.2 44.3) (end 86.2 48) (width 1) (layer B.Cu) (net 5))
 (segment (start 86.2 43.5) (end 86.2 44.3) (width 1) (layer B.Cu) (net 5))
 (segment (start 89.04 35.16) (end 89.04 31.3) (width 1) (layer B.Cu) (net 5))
 (segment (start 86.2 44.3) (end 86.2 38) (width 1) (layer B.Cu) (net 5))
 (segment (start 86.2 38) (end 89.04 35.16) (width 1) (layer B.Cu) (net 5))
 (segment (start 48.33 51.6) (end 48.34 51.61) (width 4) (layer B.Cu) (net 8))
 (segment (start 37.1 51.6) (end 48.33 51.6) (width 4) (layer B.Cu) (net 8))
 (segment (start 54.3 53.6) (end 56.3 51.6) (width 4) (layer B.Cu) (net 8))
 (segment (start 48.34 51.61) (end 50.33 53.6) (width 4) (layer B.Cu) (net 8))
 (segment (start 50.33 53.6) (end 54.3 53.6) (width 4) (layer B.Cu) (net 8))
 (segment (start 81.4 38.6) (end 81.4 36.8) (width 1) (layer B.Cu) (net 4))
 (segment (start 81.4 40.6) (end 81.4 38.6) (width 1) (layer B.Cu) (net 4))
 (segment (start 86.5 34.7) (end 86.5 31.3) (width 1) (layer B.Cu) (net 4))
 (segment (start 81.4 38.6) (end 82.6 38.6) (width 1) (layer B.Cu) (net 4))
 (segment (start 82.6 38.6) (end 86.5 34.7) (width 1) (layer B.Cu) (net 4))
 (segment (start 98.9 43.16) (end 98.9 45.7) (width 1) (layer B.Cu) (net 19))
 (segment (start 39.92 60.02) (end 39.92 61.7) (width 1) (layer B.Cu) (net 18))
 (segment (start 28.72 44.52) (end 30.9 46.7) (width 1) (layer B.Cu) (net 18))
 (segment (start 25.9 44.52) (end 28.72 44.52) (width 1) (layer B.Cu) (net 18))
 (segment (start 30.9 46.7) (end 30.9 53.5) (width 1) (layer B.Cu) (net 18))
 (segment (start 30.9 53.5) (end 36.100009 58.700009) (width 1) (layer B.Cu) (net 18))
 (segment (start 36.100009 58.700009) (end 38.600009 58.700009) (width 1) (layer B.Cu) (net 18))
 (segment (start 38.600009 58.700009) (end 39.92 60.02) (width 1) (layer B.Cu) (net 18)))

